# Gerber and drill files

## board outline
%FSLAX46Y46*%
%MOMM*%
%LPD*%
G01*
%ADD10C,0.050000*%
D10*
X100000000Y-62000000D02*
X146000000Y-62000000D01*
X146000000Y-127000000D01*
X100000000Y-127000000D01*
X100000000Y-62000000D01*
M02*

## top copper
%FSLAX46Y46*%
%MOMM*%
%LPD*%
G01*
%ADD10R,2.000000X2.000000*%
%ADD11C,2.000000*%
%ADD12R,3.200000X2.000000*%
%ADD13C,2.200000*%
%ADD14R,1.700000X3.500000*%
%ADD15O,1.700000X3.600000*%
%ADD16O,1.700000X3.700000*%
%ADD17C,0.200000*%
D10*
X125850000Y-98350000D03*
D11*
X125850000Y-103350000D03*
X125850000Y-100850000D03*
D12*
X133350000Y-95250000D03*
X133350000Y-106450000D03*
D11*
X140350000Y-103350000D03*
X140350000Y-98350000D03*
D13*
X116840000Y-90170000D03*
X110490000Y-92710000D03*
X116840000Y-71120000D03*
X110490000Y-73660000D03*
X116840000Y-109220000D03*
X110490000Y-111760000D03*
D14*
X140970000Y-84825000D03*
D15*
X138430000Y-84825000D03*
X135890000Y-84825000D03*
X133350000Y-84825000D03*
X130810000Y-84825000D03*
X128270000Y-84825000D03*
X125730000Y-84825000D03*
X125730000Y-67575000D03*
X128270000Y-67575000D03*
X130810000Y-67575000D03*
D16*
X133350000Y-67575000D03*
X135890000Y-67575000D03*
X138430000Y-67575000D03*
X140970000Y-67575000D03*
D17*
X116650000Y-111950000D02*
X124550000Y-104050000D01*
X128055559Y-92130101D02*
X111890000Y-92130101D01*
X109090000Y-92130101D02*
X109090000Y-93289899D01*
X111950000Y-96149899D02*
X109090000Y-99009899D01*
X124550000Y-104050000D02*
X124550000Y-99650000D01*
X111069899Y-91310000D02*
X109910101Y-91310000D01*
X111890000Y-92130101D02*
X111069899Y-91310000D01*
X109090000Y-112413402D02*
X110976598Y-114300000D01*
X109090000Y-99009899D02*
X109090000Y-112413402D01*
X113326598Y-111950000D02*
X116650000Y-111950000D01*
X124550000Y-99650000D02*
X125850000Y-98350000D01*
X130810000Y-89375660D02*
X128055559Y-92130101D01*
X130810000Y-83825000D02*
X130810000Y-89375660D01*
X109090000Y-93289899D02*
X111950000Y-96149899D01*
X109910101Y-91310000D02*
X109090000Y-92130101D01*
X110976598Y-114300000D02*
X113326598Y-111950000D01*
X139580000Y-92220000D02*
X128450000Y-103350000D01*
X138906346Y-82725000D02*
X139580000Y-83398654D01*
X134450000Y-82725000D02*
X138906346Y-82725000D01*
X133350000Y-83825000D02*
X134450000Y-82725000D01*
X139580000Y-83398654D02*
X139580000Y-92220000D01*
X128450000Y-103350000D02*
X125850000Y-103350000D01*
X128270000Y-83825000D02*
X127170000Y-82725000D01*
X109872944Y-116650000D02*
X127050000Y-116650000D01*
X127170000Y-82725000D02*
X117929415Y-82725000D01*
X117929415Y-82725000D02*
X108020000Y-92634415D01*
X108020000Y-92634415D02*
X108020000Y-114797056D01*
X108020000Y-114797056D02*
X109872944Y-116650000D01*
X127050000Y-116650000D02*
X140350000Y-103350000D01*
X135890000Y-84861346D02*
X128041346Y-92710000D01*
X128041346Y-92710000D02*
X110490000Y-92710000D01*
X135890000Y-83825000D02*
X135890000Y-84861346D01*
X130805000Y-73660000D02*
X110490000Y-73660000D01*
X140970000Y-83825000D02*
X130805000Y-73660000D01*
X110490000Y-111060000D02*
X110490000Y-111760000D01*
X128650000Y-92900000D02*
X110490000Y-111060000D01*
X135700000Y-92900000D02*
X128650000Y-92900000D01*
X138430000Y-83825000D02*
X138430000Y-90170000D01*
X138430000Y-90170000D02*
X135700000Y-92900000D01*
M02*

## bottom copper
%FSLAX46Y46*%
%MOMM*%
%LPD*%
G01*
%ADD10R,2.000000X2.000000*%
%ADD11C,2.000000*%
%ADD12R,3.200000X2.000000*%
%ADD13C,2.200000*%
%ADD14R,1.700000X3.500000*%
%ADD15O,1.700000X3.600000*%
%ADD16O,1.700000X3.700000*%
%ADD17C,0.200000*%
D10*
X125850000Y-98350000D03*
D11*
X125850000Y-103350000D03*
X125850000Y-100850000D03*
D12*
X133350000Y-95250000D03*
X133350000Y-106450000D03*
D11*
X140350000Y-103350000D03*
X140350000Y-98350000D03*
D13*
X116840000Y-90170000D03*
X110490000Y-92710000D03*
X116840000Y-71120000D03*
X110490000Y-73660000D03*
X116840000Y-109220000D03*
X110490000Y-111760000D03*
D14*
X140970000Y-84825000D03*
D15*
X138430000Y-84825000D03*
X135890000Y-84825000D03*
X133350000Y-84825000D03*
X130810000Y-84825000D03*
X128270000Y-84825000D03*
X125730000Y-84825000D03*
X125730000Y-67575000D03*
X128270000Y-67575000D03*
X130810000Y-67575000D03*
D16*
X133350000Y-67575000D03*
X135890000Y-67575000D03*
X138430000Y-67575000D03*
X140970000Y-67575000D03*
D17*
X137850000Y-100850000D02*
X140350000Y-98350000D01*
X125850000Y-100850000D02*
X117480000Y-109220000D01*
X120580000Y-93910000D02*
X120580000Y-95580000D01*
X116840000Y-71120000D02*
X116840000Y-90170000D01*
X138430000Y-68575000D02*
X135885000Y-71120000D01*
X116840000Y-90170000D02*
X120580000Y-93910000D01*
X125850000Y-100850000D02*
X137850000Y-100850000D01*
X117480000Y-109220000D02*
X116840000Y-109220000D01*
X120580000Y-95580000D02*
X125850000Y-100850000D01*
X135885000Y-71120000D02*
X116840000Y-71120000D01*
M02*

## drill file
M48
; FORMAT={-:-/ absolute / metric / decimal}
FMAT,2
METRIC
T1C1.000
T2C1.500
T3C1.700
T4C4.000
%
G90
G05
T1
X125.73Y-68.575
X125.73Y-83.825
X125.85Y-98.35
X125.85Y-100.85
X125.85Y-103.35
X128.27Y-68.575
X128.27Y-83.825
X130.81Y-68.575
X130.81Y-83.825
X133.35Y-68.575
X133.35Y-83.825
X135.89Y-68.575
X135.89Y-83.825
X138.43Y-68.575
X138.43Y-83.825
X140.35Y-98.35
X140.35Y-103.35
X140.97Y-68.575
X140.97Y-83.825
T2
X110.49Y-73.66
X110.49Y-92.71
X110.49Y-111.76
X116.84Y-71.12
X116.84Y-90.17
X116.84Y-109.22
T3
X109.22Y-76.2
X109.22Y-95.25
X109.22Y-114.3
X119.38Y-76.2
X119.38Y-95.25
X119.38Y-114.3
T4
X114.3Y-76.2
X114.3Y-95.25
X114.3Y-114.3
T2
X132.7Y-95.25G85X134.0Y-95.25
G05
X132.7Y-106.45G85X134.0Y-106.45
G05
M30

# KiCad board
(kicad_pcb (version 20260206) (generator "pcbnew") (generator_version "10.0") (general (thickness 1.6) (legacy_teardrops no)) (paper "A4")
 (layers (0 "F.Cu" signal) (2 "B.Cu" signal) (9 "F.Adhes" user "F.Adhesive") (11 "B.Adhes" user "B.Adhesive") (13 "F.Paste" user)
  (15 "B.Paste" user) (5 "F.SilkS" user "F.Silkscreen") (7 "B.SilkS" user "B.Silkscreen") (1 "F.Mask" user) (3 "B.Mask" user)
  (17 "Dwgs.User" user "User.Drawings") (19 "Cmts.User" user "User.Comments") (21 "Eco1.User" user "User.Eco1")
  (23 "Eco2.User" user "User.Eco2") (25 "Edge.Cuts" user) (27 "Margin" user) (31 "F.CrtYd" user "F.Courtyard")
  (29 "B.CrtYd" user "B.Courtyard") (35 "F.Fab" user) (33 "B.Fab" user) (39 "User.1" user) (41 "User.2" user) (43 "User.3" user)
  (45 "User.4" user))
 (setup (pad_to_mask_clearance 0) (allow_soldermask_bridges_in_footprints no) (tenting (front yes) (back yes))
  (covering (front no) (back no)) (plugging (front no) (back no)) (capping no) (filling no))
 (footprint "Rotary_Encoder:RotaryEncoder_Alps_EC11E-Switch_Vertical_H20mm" (layer "F.Cu") (at 125.85 98.35)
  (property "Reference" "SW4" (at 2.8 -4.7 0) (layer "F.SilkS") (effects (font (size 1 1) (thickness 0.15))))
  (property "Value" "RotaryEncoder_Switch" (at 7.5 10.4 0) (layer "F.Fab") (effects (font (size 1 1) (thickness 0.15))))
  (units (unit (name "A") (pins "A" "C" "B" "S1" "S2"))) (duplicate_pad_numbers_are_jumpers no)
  (pad "A" thru_hole rect (at 0 0) (size 2 2) (drill 1) (layers "*.Cu" "*.Mask") (remove_unused_layers no) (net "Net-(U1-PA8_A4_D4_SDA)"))
  (pad "B" thru_hole circle (at 0 5) (size 2 2) (drill 1) (layers "*.Cu" "*.Mask") (remove_unused_layers no) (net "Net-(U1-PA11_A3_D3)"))
  (pad "C" thru_hole circle (at 0 2.5) (size 2 2) (drill 1) (layers "*.Cu" "*.Mask") (remove_unused_layers no) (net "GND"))
  (pad "MP" thru_hole rect (at 7.5 -3.1) (size 3.2 2) (drill oval 2.8 1.5) (layers "*.Cu" "*.Mask") (remove_unused_layers no))
  (pad "MP" thru_hole rect (at 7.5 8.1) (size 3.2 2) (drill oval 2.8 1.5) (layers "*.Cu" "*.Mask") (remove_unused_layers no))
  (pad "S1" thru_hole circle (at 14.5 5) (size 2 2) (drill 1) (layers "*.Cu" "*.Mask") (remove_unused_layers no)
   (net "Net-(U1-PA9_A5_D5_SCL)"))
  (pad "S2" thru_hole circle (at 14.5 0) (size 2 2) (drill 1) (layers "*.Cu" "*.Mask") (remove_unused_layers no) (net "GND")))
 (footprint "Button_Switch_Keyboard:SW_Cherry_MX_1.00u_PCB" (layer "F.Cu") (at 116.84 90.17)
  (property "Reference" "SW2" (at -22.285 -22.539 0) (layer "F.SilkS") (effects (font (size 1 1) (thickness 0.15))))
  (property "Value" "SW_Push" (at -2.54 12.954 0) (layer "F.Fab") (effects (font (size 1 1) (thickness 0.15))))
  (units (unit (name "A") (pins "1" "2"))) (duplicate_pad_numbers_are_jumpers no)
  (pad "" np_thru_hole circle (at -7.62 5.08) (size 1.7 1.7) (drill 1.7) (layers "*.Cu" "*.Mask"))
  (pad "" np_thru_hole circle (at -2.54 5.08) (size 4 4) (drill 4) (layers "*.Cu" "*.Mask"))
  (pad "" np_thru_hole circle (at 2.54 5.08) (size 1.7 1.7) (drill 1.7) (layers "*.Cu" "*.Mask"))
  (pad "1" thru_hole circle (at 0 0) (size 2.2 2.2) (drill 1.5) (layers "*.Cu" "*.Mask") (remove_unused_layers no) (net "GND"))
  (pad "2" thru_hole circle (at -6.35 2.54) (size 2.2 2.2) (drill 1.5) (layers "*.Cu" "*.Mask") (remove_unused_layers no)
   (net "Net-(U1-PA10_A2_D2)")))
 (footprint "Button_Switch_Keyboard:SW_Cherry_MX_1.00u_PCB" (layer "F.Cu") (at 116.84 71.12)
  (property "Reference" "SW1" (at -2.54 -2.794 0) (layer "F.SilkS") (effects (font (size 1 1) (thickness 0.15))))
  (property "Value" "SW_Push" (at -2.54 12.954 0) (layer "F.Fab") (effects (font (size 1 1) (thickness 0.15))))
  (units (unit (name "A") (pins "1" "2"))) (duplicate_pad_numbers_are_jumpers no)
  (pad "" np_thru_hole circle (at -7.62 5.08) (size 1.7 1.7) (drill 1.7) (layers "*.Cu" "*.Mask"))
  (pad "" np_thru_hole circle (at -2.54 5.08) (size 4 4) (drill 4) (layers "*.Cu" "*.Mask"))
  (pad "" np_thru_hole circle (at 2.54 5.08) (size 1.7 1.7) (drill 1.7) (layers "*.Cu" "*.Mask"))
  (pad "1" thru_hole circle (at 0 0) (size 2.2 2.2) (drill 1.5) (layers "*.Cu" "*.Mask") (remove_unused_layers no) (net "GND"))
  (pad "2" thru_hole circle (at -6.35 2.54) (size 2.2 2.2) (drill 1.5) (layers "*.Cu" "*.Mask") (remove_unused_layers no)
   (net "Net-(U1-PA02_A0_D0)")))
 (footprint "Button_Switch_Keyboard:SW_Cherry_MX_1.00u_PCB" (layer "F.Cu") (at 116.84 109.22)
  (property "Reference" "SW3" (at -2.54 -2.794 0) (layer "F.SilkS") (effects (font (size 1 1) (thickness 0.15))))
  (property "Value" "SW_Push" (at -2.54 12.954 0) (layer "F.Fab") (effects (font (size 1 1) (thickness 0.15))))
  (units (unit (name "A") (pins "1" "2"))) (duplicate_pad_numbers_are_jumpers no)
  (pad "" np_thru_hole circle (at -7.62 5.08) (size 1.7 1.7) (drill 1.7) (layers "*.Cu" "*.Mask"))
  (pad "" np_thru_hole circle (at -2.54 5.08) (size 4 4) (drill 4) (layers "*.Cu" "*.Mask"))
  (pad "" np_thru_hole circle (at 2.54 5.08) (size 1.7 1.7) (drill 1.7) (layers "*.Cu" "*.Mask"))
  (pad "1" thru_hole circle (at 0 0) (size 2.2 2.2) (drill 1.5) (layers "*.Cu" "*.Mask") (remove_unused_layers no) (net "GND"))
  (pad "2" thru_hole circle (at -6.35 2.54) (size 2.2 2.2) (drill 1.5) (layers "*.Cu" "*.Mask") (remove_unused_layers no)
   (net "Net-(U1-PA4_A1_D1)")))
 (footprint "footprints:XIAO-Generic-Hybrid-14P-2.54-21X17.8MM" (layer "B.Cu") (at 133.35 76.2 90)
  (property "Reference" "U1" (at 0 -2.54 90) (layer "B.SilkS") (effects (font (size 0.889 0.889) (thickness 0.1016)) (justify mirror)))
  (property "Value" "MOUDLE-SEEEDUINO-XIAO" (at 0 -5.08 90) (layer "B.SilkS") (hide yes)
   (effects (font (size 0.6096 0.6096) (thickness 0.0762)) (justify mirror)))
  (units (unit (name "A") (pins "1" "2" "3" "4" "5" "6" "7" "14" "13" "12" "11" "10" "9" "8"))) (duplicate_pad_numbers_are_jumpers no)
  (pad "1" thru_hole rect (at -7.625 7.62 90) (size 3.5 1.7) (drill 1 (offset -1 0)) (layers "*.Cu" "*.Mask") (remove_unused_layers no)
   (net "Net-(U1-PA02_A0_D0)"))
  (pad "2" thru_hole oval (at -7.625 5.08 90) (size 3.6 1.7) (drill 1 (offset -1 0)) (layers "*.Cu" "*.Mask") (remove_unused_layers no)
   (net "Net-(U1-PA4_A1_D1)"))
  (pad "3" thru_hole oval (at -7.625 2.54 90) (size 3.6 1.7) (drill 1 (offset -1 0)) (layers "*.Cu" "*.Mask") (remove_unused_layers no)
   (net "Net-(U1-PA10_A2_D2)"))
  (pad "4" thru_hole oval (at -7.625 0 90) (size 3.6 1.7) (drill 1 (offset -1 0)) (layers "*.Cu" "*.Mask") (remove_unused_layers no)
   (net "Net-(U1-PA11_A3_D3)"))
  (pad "5" thru_hole oval (at -7.625 -2.54 90) (size 3.6 1.7) (drill 1 (offset -1 0)) (layers "*.Cu" "*.Mask") (remove_unused_layers no)
   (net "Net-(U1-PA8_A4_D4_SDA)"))
  (pad "6" thru_hole oval (at -7.625 -5.08 270) (size 3.6 1.7) (drill 1 (offset 1 0)) (layers "*.Cu" "*.Mask") (remove_unused_layers no)
   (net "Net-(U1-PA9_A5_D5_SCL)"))
  (pad "7" thru_hole oval (at -7.625 -7.62 90) (size 3.6 1.7) (drill 1 (offset -1 0)) (layers "*.Cu" "*.Mask") (remove_unused_layers no)
   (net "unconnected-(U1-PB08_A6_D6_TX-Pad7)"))
  (pad "8" thru_hole oval (at 7.625 -7.62 90) (size 3.6 1.7) (drill 1 (offset 1 0)) (layers "*.Cu" "*.Mask") (remove_unused_layers no)
   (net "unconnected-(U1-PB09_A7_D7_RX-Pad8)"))
  (pad "9" thru_hole oval (at 7.625 -5.08 90) (size 3.6 1.7) (drill 1 (offset 1 0)) (layers "*.Cu" "*.Mask") (remove_unused_layers no)
   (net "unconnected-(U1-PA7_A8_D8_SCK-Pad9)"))
  (pad "10" thru_hole oval (at 7.625 -2.54 90) (size 3.6 1.7) (drill 1 (offset 1 0)) (layers "*.Cu" "*.Mask") (remove_unused_layers no)
   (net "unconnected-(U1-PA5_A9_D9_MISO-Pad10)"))
  (pad "11" thru_hole oval (at 7.625 0 90) (size 3.7 1.7) (drill 1 (offset 1 0)) (layers "*.Cu" "*.Mask") (remove_unused_layers no)
   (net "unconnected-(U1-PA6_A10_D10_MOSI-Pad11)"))
  (pad "12" thru_hole oval (at 7.625 2.54 90) (size 3.7 1.7) (drill 1 (offset 1 0)) (layers "*.Cu" "*.Mask") (remove_unused_layers no)
   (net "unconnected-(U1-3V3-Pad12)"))
  (pad "13" thru_hole oval (at 7.625 5.08 90) (size 3.7 1.7) (drill 1 (offset 1 0)) (layers "*.Cu" "*.Mask") (remove_unused_layers no)
   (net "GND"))
  (pad "14" thru_hole oval (at 7.625 7.62 90) (size 3.7 1.7) (drill 1 (offset 1 0)) (layers "*.Cu" "*.Mask") (remove_unused_layers no)
   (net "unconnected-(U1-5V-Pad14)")))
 (gr_rect (start 100 62) (end 146 127) (stroke (width 0.05) (type default)) (fill no) (layer "Edge.Cuts"))
 (segment (start 116.65 111.95) (end 124.55 104.05) (width 0.2) (layer "F.Cu") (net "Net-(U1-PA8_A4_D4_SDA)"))
 (segment (start 128.055559 92.130101) (end 111.89 92.130101) (width 0.2) (layer "F.Cu") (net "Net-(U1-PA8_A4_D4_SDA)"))
 (segment (start 109.09 92.130101) (end 109.09 93.289899) (width 0.2) (layer "F.Cu") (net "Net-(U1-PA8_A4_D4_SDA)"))
 (segment (start 111.95 96.149899) (end 109.09 99.009899) (width 0.2) (layer "F.Cu") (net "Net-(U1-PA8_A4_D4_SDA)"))
 (segment (start 124.55 104.05) (end 124.55 99.65) (width 0.2) (layer "F.Cu") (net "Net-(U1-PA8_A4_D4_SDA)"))
 (segment (start 111.069899 91.31) (end 109.910101 91.31) (width 0.2) (layer "F.Cu") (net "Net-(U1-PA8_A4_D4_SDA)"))
 (segment (start 111.89 92.130101) (end 111.069899 91.31) (width 0.2) (layer "F.Cu") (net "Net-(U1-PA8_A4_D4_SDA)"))
 (segment (start 109.09 112.413402) (end 110.976598 114.3) (width 0.2) (layer "F.Cu") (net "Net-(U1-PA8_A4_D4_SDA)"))
 (segment (start 109.09 99.009899) (end 109.09 112.413402) (width 0.2) (layer "F.Cu") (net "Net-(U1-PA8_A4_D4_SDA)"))
 (segment (start 113.326598 111.95) (end 116.65 111.95) (width 0.2) (layer "F.Cu") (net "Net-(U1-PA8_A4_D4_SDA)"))
 (segment (start 124.55 99.65) (end 125.85 98.35) (width 0.2) (layer "F.Cu") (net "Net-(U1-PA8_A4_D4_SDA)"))
 (segment (start 130.81 89.37566) (end 128.055559 92.130101) (width 0.2) (layer "F.Cu") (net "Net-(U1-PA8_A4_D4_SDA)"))
 (segment (start 130.81 83.825) (end 130.81 89.37566) (width 0.2) (layer "F.Cu") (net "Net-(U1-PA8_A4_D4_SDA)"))
 (segment (start 109.09 93.289899) (end 111.95 96.149899) (width 0.2) (layer "F.Cu") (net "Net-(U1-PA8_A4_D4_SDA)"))
 (segment (start 109.910101 91.31) (end 109.09 92.130101) (width 0.2) (layer "F.Cu") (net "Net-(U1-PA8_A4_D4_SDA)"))
 (segment (start 110.976598 114.3) (end 113.326598 111.95) (width 0.2) (layer "F.Cu") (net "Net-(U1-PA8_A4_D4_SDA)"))
 (segment (start 139.58 92.22) (end 128.45 103.35) (width 0.2) (layer "F.Cu") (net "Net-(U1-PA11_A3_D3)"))
 (segment (start 138.906346 82.725) (end 139.58 83.398654) (width 0.2) (layer "F.Cu") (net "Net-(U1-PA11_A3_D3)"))
 (segment (start 134.45 82.725) (end 138.906346 82.725) (width 0.2) (layer "F.Cu") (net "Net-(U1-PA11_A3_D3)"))
 (segment (start 133.35 83.825) (end 134.45 82.725) (width 0.2) (layer "F.Cu") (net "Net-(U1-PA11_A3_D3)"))
 (segment (start 139.58 83.398654) (end 139.58 92.22) (width 0.2) (layer "F.Cu") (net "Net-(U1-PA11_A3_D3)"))
 (segment (start 128.45 103.35) (end 125.85 103.35) (width 0.2) (layer "F.Cu") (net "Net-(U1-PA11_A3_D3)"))
 (segment (start 137.85 100.85) (end 140.35 98.35) (width 0.2) (layer "B.Cu") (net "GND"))
 (segment (start 125.85 100.85) (end 117.48 109.22) (width 0.2) (layer "B.Cu") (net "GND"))
 (segment (start 120.58 93.91) (end 120.58 95.58) (width 0.2) (layer "B.Cu") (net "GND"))
 (segment (start 116.84 71.12) (end 116.84 90.17) (width 0.2) (layer "B.Cu") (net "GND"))
 (segment (start 138.43 68.575) (end 135.885 71.12) (width 0.2) (layer "B.Cu") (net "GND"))
 (segment (start 116.84 90.17) (end 120.58 93.91) (width 0.2) (layer "B.Cu") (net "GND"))
 (segment (start 125.85 100.85) (end 137.85 100.85) (width 0.2) (layer "B.Cu") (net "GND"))
 (segment (start 117.48 109.22) (end 116.84 109.22) (width 0.2) (layer "B.Cu") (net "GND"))
 (segment (start 120.58 95.58) (end 125.85 100.85) (width 0.2) (layer "B.Cu") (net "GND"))
 (segment (start 135.885 71.12) (end 116.84 71.12) (width 0.2) (layer "B.Cu") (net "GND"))
 (segment (start 128.27 83.825) (end 127.17 82.725) (width 0.2) (layer "F.Cu") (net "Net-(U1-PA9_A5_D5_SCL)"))
 (segment (start 109.872944 116.65) (end 127.05 116.65) (width 0.2) (layer "F.Cu") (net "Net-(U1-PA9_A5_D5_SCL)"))
 (segment (start 127.17 82.725) (end 117.929415 82.725) (width 0.2) (layer "F.Cu") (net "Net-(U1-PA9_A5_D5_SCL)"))
 (segment (start 117.929415 82.725) (end 108.02 92.634415) (width 0.2) (layer "F.Cu") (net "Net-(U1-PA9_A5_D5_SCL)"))
 (segment (start 108.02 92.634415) (end 108.02 114.797056) (width 0.2) (layer "F.Cu") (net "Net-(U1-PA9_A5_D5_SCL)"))
 (segment (start 108.02 114.797056) (end 109.872944 116.65) (width 0.2) (layer "F.Cu") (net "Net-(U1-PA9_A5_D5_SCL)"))
 (segment (start 127.05 116.65) (end 140.35 103.35) (width 0.2) (layer "F.Cu") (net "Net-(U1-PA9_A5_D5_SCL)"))
 (segment (start 135.89 84.861346) (end 128.041346 92.71) (width 0.2) (layer "F.Cu") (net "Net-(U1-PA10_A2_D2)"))
 (segment (start 128.041346 92.71) (end 110.49 92.71) (width 0.2) (layer "F.Cu") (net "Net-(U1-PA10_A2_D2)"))
 (segment (start 135.89 83.825) (end 135.89 84.861346) (width 0.2) (layer "F.Cu") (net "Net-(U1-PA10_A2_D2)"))
 (segment (start 130.805 73.66) (end 110.49 73.66) (width 0.2) (layer "F.Cu") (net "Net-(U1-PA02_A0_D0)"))
 (segment (start 140.97 83.825) (end 130.805 73.66) (width 0.2) (layer "F.Cu") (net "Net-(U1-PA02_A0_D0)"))
 (segment (start 110.49 111.06) (end 110.49 111.76) (width 0.2) (layer "F.Cu") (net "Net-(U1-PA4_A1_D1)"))
 (segment (start 128.65 92.9) (end 110.49 111.06) (width 0.2) (layer "F.Cu") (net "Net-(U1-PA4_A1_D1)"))
 (segment (start 135.7 92.9) (end 128.65 92.9) (width 0.2) (layer "F.Cu") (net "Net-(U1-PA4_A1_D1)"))
 (segment (start 138.43 83.825) (end 138.43 90.17) (width 0.2) (layer "F.Cu") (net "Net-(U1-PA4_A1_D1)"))
 (segment (start 138.43 90.17) (end 135.7 92.9) (width 0.2) (layer "F.Cu") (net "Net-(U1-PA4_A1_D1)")))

